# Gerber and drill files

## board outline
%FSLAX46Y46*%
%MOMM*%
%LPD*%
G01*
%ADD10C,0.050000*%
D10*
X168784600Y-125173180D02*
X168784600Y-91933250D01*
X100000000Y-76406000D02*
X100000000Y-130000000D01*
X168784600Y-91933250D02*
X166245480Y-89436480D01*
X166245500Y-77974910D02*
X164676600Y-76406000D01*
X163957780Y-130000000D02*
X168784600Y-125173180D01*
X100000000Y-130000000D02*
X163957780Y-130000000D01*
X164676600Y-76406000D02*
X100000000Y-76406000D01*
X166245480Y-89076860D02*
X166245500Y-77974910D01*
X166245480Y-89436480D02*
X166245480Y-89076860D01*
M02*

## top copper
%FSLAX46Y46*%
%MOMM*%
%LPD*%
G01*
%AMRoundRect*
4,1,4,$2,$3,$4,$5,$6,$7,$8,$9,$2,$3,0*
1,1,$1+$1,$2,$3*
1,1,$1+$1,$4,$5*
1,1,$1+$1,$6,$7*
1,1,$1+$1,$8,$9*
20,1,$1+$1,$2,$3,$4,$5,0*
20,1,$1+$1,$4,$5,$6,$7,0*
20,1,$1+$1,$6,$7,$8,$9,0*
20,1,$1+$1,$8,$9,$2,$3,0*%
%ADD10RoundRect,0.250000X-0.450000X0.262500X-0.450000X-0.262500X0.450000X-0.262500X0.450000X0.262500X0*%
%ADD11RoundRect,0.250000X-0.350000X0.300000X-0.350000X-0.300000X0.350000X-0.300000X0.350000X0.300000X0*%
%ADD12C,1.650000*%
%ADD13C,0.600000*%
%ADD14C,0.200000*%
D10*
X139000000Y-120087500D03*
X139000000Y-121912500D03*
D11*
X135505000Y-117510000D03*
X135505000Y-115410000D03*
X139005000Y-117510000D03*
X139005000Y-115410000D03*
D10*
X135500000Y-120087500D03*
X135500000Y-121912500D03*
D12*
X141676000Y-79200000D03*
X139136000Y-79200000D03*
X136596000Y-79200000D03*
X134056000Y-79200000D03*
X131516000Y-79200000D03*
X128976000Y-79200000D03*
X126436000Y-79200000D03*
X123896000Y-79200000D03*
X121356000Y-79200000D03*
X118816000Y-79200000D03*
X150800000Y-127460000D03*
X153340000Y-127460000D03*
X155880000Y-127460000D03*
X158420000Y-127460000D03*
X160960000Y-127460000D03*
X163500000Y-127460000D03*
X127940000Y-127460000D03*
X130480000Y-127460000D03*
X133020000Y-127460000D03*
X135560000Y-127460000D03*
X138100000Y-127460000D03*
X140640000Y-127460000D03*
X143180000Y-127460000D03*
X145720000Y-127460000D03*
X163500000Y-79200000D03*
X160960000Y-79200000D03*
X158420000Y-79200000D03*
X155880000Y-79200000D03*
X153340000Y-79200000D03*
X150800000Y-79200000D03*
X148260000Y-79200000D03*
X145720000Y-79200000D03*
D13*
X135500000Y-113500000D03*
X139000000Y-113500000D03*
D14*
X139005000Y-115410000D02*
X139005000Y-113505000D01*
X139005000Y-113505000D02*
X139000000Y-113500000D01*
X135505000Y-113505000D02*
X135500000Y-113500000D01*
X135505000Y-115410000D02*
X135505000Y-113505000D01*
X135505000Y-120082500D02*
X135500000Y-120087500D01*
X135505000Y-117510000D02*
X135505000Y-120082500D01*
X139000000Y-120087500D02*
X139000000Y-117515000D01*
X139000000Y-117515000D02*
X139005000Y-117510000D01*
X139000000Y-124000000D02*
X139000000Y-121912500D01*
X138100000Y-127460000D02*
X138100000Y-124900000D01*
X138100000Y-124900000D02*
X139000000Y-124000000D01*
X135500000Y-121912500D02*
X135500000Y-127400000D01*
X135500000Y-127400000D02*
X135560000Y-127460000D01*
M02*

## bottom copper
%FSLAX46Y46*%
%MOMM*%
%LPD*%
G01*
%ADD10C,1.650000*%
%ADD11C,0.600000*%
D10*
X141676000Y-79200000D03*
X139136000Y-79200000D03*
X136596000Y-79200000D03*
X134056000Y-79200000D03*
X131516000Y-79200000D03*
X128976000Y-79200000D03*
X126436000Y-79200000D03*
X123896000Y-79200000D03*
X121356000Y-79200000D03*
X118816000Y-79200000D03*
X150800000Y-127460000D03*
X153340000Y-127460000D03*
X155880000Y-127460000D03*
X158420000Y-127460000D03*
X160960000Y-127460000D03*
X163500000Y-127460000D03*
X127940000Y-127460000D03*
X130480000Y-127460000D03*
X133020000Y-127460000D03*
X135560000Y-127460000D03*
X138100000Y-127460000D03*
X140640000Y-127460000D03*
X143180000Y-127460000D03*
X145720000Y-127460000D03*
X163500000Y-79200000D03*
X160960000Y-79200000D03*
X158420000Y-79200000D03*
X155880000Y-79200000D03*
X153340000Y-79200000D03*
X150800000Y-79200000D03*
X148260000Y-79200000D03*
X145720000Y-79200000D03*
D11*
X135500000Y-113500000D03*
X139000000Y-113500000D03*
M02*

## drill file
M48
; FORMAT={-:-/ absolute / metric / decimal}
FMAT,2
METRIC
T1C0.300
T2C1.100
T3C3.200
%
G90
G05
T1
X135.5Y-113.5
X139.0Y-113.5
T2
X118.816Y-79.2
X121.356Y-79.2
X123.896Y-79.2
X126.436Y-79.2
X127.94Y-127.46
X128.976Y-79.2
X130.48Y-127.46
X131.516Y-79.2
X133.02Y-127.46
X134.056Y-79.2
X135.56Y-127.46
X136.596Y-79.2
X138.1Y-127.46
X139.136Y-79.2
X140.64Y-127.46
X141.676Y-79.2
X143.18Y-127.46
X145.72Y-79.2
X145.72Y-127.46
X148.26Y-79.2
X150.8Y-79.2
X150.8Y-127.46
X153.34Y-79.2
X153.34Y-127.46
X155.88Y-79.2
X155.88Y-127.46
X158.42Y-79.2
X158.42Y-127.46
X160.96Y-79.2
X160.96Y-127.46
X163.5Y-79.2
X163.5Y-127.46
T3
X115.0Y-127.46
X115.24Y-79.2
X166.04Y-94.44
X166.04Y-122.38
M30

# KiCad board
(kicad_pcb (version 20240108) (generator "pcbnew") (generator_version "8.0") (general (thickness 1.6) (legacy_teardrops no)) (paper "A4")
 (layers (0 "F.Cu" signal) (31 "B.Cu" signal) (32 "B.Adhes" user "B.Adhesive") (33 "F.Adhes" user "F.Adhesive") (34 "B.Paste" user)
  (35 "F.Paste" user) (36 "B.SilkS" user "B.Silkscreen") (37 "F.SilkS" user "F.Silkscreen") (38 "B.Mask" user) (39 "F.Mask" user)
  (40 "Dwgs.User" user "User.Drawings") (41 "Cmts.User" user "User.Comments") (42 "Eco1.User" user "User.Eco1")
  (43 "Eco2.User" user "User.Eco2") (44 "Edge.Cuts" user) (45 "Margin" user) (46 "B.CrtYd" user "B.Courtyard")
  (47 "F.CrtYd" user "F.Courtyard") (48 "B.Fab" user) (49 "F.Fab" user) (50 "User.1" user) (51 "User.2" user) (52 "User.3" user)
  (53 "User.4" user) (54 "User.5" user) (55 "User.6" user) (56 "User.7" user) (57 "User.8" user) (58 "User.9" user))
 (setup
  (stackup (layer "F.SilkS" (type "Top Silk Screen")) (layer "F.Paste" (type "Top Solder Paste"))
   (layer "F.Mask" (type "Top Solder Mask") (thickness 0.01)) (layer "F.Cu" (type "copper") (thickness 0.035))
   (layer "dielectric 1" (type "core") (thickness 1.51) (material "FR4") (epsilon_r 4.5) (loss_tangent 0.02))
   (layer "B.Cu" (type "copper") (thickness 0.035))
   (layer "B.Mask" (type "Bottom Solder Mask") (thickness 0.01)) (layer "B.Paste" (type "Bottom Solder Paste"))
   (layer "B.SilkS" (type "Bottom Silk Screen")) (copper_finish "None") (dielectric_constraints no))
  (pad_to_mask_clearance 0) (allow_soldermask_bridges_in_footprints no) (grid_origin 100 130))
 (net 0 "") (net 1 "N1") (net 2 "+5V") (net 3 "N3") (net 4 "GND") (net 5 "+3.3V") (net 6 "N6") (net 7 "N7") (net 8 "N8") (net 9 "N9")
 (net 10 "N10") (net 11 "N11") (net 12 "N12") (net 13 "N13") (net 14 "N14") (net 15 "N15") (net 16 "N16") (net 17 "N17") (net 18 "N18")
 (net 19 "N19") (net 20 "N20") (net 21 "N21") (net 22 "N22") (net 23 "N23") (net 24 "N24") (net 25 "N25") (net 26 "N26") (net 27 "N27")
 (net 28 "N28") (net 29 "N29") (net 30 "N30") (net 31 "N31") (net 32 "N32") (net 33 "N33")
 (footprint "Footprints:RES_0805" (layer "F.Cu") (at 139 121 -90)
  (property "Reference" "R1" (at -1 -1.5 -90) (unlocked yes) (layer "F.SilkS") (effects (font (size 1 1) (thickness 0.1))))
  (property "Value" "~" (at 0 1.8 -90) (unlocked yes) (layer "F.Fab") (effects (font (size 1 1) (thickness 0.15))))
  (pad "1" smd roundrect (at -0.9125 0 270) (size 1.025 1.4) (layers "F.Cu" "F.Paste" "F.Mask") (roundrect_rratio 0.243902) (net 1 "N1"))
  (pad "2" smd roundrect (at 0.9125 0 270) (size 1.025 1.4) (layers "F.Cu" "F.Paste" "F.Mask") (roundrect_rratio 0.243902) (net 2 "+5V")))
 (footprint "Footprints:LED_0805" (layer "F.Cu") (at 135.5 116.5 -90)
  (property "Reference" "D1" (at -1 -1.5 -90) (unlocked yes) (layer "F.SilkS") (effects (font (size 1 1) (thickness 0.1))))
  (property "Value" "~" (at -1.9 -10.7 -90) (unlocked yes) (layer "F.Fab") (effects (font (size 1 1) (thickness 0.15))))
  (pad "A" smd roundrect (at 1.01 -0.005 270) (size 1.1 1.2) (layers "F.Cu" "F.Paste" "F.Mask") (roundrect_rratio 0.2272727273) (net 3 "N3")
   (solder_mask_margin 0.102))
  (pad "K" smd roundrect (at -1.09 -0.005 270) (size 1.1 1.2) (layers "F.Cu" "F.Paste" "F.Mask") (roundrect_rratio 0.2272727273)
   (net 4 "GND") (solder_mask_margin 0.102)))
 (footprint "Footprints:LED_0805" (layer "F.Cu") (at 139 116.5 -90)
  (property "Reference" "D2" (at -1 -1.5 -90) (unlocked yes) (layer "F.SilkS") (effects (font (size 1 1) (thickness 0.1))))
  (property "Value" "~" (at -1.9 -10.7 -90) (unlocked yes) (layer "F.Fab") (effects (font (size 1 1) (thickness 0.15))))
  (pad "A" smd roundrect (at 1.01 -0.005 270) (size 1.1 1.2) (layers "F.Cu" "F.Paste" "F.Mask") (roundrect_rratio 0.2272727273) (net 1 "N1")
   (solder_mask_margin 0.102))
  (pad "K" smd roundrect (at -1.09 -0.005 270) (size 1.1 1.2) (layers "F.Cu" "F.Paste" "F.Mask") (roundrect_rratio 0.2272727273)
   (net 4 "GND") (solder_mask_margin 0.102)))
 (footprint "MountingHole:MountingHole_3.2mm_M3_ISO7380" (layer "F.Cu") (at 115 127.46)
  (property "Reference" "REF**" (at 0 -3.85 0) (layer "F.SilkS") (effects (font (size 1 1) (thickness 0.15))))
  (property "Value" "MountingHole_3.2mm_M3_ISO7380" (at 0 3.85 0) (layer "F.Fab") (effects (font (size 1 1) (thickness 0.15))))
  (pad "" np_thru_hole circle (at 0 0) (size 3.2 3.2) (drill 3.2) (layers "F&B.Cu" "*.Mask")))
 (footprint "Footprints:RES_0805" (layer "F.Cu") (at 135.5 121 -90)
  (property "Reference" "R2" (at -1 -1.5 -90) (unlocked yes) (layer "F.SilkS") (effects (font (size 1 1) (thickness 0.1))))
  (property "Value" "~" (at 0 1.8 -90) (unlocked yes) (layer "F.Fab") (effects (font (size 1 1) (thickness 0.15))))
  (pad "1" smd roundrect (at -0.9125 0 270) (size 1.025 1.4) (layers "F.Cu" "F.Paste" "F.Mask") (roundrect_rratio 0.243902) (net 3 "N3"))
  (pad "2" smd roundrect (at 0.9125 0 270) (size 1.025 1.4) (layers "F.Cu" "F.Paste" "F.Mask") (roundrect_rratio 0.243902) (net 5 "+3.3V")))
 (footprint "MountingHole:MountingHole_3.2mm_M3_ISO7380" (layer "F.Cu") (at 166.04 94.44)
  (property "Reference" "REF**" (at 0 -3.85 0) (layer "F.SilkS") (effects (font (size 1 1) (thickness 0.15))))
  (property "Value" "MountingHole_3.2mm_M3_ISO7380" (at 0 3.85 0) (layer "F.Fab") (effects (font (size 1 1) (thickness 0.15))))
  (pad "" np_thru_hole circle (at 0 0) (size 3.2 3.2) (drill 3.2) (layers "*.Cu" "*.Mask")))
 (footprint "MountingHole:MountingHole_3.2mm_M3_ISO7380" (layer "F.Cu") (at 115.24 79.2)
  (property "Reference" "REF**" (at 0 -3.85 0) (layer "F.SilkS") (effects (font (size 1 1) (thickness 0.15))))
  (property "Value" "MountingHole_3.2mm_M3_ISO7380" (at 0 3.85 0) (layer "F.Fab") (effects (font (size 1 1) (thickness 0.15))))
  (pad "" np_thru_hole circle (at 0 0) (size 3.2 3.2) (drill 3.2) (layers "*.Cu" "*.Mask")))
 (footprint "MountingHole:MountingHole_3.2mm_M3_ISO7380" (layer "F.Cu") (at 166.04 122.38)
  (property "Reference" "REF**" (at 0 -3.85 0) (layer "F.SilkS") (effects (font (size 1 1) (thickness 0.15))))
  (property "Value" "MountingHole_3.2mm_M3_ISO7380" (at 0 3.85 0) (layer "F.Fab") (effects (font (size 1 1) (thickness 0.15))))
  (pad "" np_thru_hole circle (at 0 0) (size 3.2 3.2) (drill 3.2) (layers "*.Cu" "*.Mask")))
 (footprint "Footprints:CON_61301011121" (layer "B.Cu") (at 130.226 79.2 180)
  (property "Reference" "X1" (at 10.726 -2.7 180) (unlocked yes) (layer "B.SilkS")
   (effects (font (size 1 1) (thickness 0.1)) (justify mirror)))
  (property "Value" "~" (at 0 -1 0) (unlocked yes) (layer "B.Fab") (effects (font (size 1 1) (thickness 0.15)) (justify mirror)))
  (pad "1" thru_hole circle (at -11.45 0 180) (size 1.65 1.65) (drill 1.1) (layers "*.Cu" "*.Mask") (remove_unused_layers no) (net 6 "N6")
   (solder_mask_margin 0.102))
  (pad "2" thru_hole circle (at -8.91 0 180) (size 1.65 1.65) (drill 1.1) (layers "*.Cu" "*.Mask") (remove_unused_layers no) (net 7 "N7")
   (solder_mask_margin 0.102))
  (pad "3" thru_hole circle (at -6.37 0 180) (size 1.65 1.65) (drill 1.1) (layers "*.Cu" "*.Mask") (remove_unused_layers no) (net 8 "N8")
   (solder_mask_margin 0.102))
  (pad "4" thru_hole circle (at -3.83 0 180) (size 1.65 1.65) (drill 1.1) (layers "*.Cu" "*.Mask") (remove_unused_layers no) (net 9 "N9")
   (solder_mask_margin 0.102))
  (pad "5" thru_hole circle (at -1.29 0 180) (size 1.65 1.65) (drill 1.1) (layers "*.Cu" "*.Mask") (remove_unused_layers no) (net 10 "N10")
   (solder_mask_margin 0.102))
  (pad "6" thru_hole circle (at 1.25 0 180) (size 1.65 1.65) (drill 1.1) (layers "*.Cu" "*.Mask") (remove_unused_layers no) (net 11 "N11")
   (solder_mask_margin 0.102))
  (pad "7" thru_hole circle (at 3.79 0 180) (size 1.65 1.65) (drill 1.1) (layers "*.Cu" "*.Mask") (remove_unused_layers no) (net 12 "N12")
   (solder_mask_margin 0.102))
  (pad "8" thru_hole circle (at 6.33 0 180) (size 1.65 1.65) (drill 1.1) (layers "*.Cu" "*.Mask") (remove_unused_layers no) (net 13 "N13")
   (solder_mask_margin 0.102))
  (pad "9" thru_hole circle (at 8.87 0 180) (size 1.65 1.65) (drill 1.1) (layers "*.Cu" "*.Mask") (remove_unused_layers no) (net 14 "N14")
   (solder_mask_margin 0.102))
  (pad "10" thru_hole circle (at 11.41 0 180) (size 1.65 1.65) (drill 1.1) (layers "*.Cu" "*.Mask") (remove_unused_layers no) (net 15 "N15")
   (solder_mask_margin 0.102)))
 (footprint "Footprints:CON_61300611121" (layer "B.Cu") (at 157.15 127.46)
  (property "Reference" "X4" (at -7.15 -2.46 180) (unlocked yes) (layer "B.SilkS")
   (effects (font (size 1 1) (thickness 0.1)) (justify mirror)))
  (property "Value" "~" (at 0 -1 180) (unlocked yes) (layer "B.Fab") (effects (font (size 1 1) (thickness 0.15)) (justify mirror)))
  (pad "1" thru_hole circle (at -6.35 0) (size 1.65 1.65) (drill 1.1) (layers "*.Cu" "*.Mask") (remove_unused_layers no) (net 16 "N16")
   (solder_mask_margin 0.102))
  (pad "2" thru_hole circle (at -3.81 0) (size 1.65 1.65) (drill 1.1) (layers "*.Cu" "*.Mask") (remove_unused_layers no) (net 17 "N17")
   (solder_mask_margin 0.102))
  (pad "3" thru_hole circle (at -1.27 0) (size 1.65 1.65) (drill 1.1) (layers "*.Cu" "*.Mask") (remove_unused_layers no) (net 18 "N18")
   (solder_mask_margin 0.102))
  (pad "4" thru_hole circle (at 1.27 0) (size 1.65 1.65) (drill 1.1) (layers "*.Cu" "*.Mask") (remove_unused_layers no) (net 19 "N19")
   (solder_mask_margin 0.102))
  (pad "5" thru_hole circle (at 3.81 0) (size 1.65 1.65) (drill 1.1) (layers "*.Cu" "*.Mask") (remove_unused_layers no) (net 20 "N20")
   (solder_mask_margin 0.102))
  (pad "6" thru_hole circle (at 6.35 0) (size 1.65 1.65) (drill 1.1) (layers "*.Cu" "*.Mask") (remove_unused_layers no) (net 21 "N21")
   (solder_mask_margin 0.102)))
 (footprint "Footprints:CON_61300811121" (layer "B.Cu") (at 136.83 127.46)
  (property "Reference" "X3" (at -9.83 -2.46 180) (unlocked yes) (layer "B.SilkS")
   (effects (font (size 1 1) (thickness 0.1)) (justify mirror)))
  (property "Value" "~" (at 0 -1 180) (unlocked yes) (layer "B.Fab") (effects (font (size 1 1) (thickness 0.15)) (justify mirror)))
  (pad "1" thru_hole circle (at -8.89 0) (size 1.65 1.65) (drill 1.1) (layers "*.Cu" "*.Mask") (remove_unused_layers no) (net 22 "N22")
   (solder_mask_margin 0.102))
  (pad "2" thru_hole circle (at -6.35 0) (size 1.65 1.65) (drill 1.1) (layers "*.Cu" "*.Mask") (remove_unused_layers no) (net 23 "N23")
   (solder_mask_margin 0.102))
  (pad "3" thru_hole circle (at -3.81 0) (size 1.65 1.65) (drill 1.1) (layers "*.Cu" "*.Mask") (remove_unused_layers no) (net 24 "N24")
   (solder_mask_margin 0.102))
  (pad "4" thru_hole circle (at -1.27 0) (size 1.65 1.65) (drill 1.1) (layers "*.Cu" "*.Mask") (remove_unused_layers no) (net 5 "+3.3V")
   (solder_mask_margin 0.102))
  (pad "5" thru_hole circle (at 1.27 0) (size 1.65 1.65) (drill 1.1) (layers "*.Cu" "*.Mask") (remove_unused_layers no) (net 2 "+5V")
   (solder_mask_margin 0.102))
  (pad "6" thru_hole circle (at 3.81 0) (size 1.65 1.65) (drill 1.1) (layers "*.Cu" "*.Mask") (remove_unused_layers no) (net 4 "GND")
   (solder_mask_margin 0.102))
  (pad "7" thru_hole circle (at 6.35 0) (size 1.65 1.65) (drill 1.1) (layers "*.Cu" "*.Mask") (remove_unused_layers no) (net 4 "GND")
   (solder_mask_margin 0.102))
  (pad "8" thru_hole circle (at 8.89 0) (size 1.65 1.65) (drill 1.1) (layers "*.Cu" "*.Mask") (remove_unused_layers no) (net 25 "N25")
   (solder_mask_margin 0.102)))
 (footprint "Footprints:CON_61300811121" (layer "B.Cu") (at 154.61 79.2 180)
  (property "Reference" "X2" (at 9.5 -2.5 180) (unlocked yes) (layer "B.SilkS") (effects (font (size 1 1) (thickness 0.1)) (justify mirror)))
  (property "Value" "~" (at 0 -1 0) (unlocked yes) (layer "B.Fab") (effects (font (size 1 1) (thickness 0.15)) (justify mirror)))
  (pad "1" thru_hole circle (at -8.89 0 180) (size 1.65 1.65) (drill 1.1) (layers "*.Cu" "*.Mask") (remove_unused_layers no) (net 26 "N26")
   (solder_mask_margin 0.102))
  (pad "2" thru_hole circle (at -6.35 0 180) (size 1.65 1.65) (drill 1.1) (layers "*.Cu" "*.Mask") (remove_unused_layers no) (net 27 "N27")
   (solder_mask_margin 0.102))
  (pad "3" thru_hole circle (at -3.81 0 180) (size 1.65 1.65) (drill 1.1) (layers "*.Cu" "*.Mask") (remove_unused_layers no) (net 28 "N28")
   (solder_mask_margin 0.102))
  (pad "4" thru_hole circle (at -1.27 0 180) (size 1.65 1.65) (drill 1.1) (layers "*.Cu" "*.Mask") (remove_unused_layers no) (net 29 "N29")
   (solder_mask_margin 0.102))
  (pad "5" thru_hole circle (at 1.27 0 180) (size 1.65 1.65) (drill 1.1) (layers "*.Cu" "*.Mask") (remove_unused_layers no) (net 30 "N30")
   (solder_mask_margin 0.102))
  (pad "6" thru_hole circle (at 3.81 0 180) (size 1.65 1.65) (drill 1.1) (layers "*.Cu" "*.Mask") (remove_unused_layers no) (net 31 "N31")
   (solder_mask_margin 0.102))
  (pad "7" thru_hole circle (at 6.35 0 180) (size 1.65 1.65) (drill 1.1) (layers "*.Cu" "*.Mask") (remove_unused_layers no) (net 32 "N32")
   (solder_mask_margin 0.102))
  (pad "8" thru_hole circle (at 8.89 0 180) (size 1.65 1.65) (drill 1.1) (layers "*.Cu" "*.Mask") (remove_unused_layers no) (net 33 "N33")
   (solder_mask_margin 0.102)))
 (gr_line (start 168.7846 125.17318) (end 168.7846 91.93325) (stroke (width 0.05) (type solid)) (layer "Edge.Cuts"))
 (gr_line (start 100 76.406) (end 100 130) (stroke (width 0.05) (type solid)) (layer "Edge.Cuts"))
 (gr_line (start 168.7846 91.93325) (end 166.24548 89.43648) (stroke (width 0.05) (type solid)) (layer "Edge.Cuts"))
 (gr_line (start 166.2455 77.97491) (end 164.6766 76.406) (stroke (width 0.05) (type solid)) (layer "Edge.Cuts"))
 (gr_line (start 163.95778 130) (end 168.7846 125.17318) (stroke (width 0.05) (type solid)) (layer "Edge.Cuts"))
 (gr_line (start 100 130) (end 163.95778 130) (stroke (width 0.05) (type solid)) (layer "Edge.Cuts"))
 (gr_line (start 164.6766 76.406) (end 100 76.406) (stroke (width 0.05) (type solid)) (layer "Edge.Cuts"))
 (gr_line (start 166.24548 89.07686) (end 166.2455 77.97491) (stroke (width 0.05) (type solid)) (layer "Edge.Cuts"))
 (gr_line (start 166.24548 89.43648) (end 166.24548 89.07686) (stroke (width 0.05) (type solid)) (layer "Edge.Cuts"))
 (segment (start 139.005 115.41) (end 139.005 113.505) (width 0.2) (layer "F.Cu") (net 4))
 (segment (start 139.005 113.505) (end 139 113.5) (width 0.2) (layer "F.Cu") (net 4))
 (segment (start 135.505 113.505) (end 135.5 113.5) (width 0.2) (layer "F.Cu") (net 4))
 (segment (start 135.505 115.41) (end 135.505 113.505) (width 0.2) (layer "F.Cu") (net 4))
 (via (at 135.5 113.5) (size 0.6) (drill 0.3) (layers "F.Cu" "B.Cu") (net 4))
 (via (at 139 113.5) (size 0.6) (drill 0.3) (layers "F.Cu" "B.Cu") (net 4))
 (segment (start 135.505 120.0825) (end 135.5 120.0875) (width 0.2) (layer "F.Cu") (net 3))
 (segment (start 135.505 117.51) (end 135.505 120.0825) (width 0.2) (layer "F.Cu") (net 3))
 (segment (start 139 120.0875) (end 139 117.515) (width 0.2) (layer "F.Cu") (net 1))
 (segment (start 139 117.515) (end 139.005 117.51) (width 0.2) (layer "F.Cu") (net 1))
 (segment (start 139 124) (end 139 121.9125) (width 0.2) (layer "F.Cu") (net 2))
 (segment (start 138.1 127.46) (end 138.1 124.9) (width 0.2) (layer "F.Cu") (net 2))
 (segment (start 138.1 124.9) (end 139 124) (width 0.2) (layer "F.Cu") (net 2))
 (segment (start 135.5 121.9125) (end 135.5 127.4) (width 0.2) (layer "F.Cu") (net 5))
 (segment (start 135.5 127.4) (end 135.56 127.46) (width 0.2) (layer "F.Cu") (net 5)))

